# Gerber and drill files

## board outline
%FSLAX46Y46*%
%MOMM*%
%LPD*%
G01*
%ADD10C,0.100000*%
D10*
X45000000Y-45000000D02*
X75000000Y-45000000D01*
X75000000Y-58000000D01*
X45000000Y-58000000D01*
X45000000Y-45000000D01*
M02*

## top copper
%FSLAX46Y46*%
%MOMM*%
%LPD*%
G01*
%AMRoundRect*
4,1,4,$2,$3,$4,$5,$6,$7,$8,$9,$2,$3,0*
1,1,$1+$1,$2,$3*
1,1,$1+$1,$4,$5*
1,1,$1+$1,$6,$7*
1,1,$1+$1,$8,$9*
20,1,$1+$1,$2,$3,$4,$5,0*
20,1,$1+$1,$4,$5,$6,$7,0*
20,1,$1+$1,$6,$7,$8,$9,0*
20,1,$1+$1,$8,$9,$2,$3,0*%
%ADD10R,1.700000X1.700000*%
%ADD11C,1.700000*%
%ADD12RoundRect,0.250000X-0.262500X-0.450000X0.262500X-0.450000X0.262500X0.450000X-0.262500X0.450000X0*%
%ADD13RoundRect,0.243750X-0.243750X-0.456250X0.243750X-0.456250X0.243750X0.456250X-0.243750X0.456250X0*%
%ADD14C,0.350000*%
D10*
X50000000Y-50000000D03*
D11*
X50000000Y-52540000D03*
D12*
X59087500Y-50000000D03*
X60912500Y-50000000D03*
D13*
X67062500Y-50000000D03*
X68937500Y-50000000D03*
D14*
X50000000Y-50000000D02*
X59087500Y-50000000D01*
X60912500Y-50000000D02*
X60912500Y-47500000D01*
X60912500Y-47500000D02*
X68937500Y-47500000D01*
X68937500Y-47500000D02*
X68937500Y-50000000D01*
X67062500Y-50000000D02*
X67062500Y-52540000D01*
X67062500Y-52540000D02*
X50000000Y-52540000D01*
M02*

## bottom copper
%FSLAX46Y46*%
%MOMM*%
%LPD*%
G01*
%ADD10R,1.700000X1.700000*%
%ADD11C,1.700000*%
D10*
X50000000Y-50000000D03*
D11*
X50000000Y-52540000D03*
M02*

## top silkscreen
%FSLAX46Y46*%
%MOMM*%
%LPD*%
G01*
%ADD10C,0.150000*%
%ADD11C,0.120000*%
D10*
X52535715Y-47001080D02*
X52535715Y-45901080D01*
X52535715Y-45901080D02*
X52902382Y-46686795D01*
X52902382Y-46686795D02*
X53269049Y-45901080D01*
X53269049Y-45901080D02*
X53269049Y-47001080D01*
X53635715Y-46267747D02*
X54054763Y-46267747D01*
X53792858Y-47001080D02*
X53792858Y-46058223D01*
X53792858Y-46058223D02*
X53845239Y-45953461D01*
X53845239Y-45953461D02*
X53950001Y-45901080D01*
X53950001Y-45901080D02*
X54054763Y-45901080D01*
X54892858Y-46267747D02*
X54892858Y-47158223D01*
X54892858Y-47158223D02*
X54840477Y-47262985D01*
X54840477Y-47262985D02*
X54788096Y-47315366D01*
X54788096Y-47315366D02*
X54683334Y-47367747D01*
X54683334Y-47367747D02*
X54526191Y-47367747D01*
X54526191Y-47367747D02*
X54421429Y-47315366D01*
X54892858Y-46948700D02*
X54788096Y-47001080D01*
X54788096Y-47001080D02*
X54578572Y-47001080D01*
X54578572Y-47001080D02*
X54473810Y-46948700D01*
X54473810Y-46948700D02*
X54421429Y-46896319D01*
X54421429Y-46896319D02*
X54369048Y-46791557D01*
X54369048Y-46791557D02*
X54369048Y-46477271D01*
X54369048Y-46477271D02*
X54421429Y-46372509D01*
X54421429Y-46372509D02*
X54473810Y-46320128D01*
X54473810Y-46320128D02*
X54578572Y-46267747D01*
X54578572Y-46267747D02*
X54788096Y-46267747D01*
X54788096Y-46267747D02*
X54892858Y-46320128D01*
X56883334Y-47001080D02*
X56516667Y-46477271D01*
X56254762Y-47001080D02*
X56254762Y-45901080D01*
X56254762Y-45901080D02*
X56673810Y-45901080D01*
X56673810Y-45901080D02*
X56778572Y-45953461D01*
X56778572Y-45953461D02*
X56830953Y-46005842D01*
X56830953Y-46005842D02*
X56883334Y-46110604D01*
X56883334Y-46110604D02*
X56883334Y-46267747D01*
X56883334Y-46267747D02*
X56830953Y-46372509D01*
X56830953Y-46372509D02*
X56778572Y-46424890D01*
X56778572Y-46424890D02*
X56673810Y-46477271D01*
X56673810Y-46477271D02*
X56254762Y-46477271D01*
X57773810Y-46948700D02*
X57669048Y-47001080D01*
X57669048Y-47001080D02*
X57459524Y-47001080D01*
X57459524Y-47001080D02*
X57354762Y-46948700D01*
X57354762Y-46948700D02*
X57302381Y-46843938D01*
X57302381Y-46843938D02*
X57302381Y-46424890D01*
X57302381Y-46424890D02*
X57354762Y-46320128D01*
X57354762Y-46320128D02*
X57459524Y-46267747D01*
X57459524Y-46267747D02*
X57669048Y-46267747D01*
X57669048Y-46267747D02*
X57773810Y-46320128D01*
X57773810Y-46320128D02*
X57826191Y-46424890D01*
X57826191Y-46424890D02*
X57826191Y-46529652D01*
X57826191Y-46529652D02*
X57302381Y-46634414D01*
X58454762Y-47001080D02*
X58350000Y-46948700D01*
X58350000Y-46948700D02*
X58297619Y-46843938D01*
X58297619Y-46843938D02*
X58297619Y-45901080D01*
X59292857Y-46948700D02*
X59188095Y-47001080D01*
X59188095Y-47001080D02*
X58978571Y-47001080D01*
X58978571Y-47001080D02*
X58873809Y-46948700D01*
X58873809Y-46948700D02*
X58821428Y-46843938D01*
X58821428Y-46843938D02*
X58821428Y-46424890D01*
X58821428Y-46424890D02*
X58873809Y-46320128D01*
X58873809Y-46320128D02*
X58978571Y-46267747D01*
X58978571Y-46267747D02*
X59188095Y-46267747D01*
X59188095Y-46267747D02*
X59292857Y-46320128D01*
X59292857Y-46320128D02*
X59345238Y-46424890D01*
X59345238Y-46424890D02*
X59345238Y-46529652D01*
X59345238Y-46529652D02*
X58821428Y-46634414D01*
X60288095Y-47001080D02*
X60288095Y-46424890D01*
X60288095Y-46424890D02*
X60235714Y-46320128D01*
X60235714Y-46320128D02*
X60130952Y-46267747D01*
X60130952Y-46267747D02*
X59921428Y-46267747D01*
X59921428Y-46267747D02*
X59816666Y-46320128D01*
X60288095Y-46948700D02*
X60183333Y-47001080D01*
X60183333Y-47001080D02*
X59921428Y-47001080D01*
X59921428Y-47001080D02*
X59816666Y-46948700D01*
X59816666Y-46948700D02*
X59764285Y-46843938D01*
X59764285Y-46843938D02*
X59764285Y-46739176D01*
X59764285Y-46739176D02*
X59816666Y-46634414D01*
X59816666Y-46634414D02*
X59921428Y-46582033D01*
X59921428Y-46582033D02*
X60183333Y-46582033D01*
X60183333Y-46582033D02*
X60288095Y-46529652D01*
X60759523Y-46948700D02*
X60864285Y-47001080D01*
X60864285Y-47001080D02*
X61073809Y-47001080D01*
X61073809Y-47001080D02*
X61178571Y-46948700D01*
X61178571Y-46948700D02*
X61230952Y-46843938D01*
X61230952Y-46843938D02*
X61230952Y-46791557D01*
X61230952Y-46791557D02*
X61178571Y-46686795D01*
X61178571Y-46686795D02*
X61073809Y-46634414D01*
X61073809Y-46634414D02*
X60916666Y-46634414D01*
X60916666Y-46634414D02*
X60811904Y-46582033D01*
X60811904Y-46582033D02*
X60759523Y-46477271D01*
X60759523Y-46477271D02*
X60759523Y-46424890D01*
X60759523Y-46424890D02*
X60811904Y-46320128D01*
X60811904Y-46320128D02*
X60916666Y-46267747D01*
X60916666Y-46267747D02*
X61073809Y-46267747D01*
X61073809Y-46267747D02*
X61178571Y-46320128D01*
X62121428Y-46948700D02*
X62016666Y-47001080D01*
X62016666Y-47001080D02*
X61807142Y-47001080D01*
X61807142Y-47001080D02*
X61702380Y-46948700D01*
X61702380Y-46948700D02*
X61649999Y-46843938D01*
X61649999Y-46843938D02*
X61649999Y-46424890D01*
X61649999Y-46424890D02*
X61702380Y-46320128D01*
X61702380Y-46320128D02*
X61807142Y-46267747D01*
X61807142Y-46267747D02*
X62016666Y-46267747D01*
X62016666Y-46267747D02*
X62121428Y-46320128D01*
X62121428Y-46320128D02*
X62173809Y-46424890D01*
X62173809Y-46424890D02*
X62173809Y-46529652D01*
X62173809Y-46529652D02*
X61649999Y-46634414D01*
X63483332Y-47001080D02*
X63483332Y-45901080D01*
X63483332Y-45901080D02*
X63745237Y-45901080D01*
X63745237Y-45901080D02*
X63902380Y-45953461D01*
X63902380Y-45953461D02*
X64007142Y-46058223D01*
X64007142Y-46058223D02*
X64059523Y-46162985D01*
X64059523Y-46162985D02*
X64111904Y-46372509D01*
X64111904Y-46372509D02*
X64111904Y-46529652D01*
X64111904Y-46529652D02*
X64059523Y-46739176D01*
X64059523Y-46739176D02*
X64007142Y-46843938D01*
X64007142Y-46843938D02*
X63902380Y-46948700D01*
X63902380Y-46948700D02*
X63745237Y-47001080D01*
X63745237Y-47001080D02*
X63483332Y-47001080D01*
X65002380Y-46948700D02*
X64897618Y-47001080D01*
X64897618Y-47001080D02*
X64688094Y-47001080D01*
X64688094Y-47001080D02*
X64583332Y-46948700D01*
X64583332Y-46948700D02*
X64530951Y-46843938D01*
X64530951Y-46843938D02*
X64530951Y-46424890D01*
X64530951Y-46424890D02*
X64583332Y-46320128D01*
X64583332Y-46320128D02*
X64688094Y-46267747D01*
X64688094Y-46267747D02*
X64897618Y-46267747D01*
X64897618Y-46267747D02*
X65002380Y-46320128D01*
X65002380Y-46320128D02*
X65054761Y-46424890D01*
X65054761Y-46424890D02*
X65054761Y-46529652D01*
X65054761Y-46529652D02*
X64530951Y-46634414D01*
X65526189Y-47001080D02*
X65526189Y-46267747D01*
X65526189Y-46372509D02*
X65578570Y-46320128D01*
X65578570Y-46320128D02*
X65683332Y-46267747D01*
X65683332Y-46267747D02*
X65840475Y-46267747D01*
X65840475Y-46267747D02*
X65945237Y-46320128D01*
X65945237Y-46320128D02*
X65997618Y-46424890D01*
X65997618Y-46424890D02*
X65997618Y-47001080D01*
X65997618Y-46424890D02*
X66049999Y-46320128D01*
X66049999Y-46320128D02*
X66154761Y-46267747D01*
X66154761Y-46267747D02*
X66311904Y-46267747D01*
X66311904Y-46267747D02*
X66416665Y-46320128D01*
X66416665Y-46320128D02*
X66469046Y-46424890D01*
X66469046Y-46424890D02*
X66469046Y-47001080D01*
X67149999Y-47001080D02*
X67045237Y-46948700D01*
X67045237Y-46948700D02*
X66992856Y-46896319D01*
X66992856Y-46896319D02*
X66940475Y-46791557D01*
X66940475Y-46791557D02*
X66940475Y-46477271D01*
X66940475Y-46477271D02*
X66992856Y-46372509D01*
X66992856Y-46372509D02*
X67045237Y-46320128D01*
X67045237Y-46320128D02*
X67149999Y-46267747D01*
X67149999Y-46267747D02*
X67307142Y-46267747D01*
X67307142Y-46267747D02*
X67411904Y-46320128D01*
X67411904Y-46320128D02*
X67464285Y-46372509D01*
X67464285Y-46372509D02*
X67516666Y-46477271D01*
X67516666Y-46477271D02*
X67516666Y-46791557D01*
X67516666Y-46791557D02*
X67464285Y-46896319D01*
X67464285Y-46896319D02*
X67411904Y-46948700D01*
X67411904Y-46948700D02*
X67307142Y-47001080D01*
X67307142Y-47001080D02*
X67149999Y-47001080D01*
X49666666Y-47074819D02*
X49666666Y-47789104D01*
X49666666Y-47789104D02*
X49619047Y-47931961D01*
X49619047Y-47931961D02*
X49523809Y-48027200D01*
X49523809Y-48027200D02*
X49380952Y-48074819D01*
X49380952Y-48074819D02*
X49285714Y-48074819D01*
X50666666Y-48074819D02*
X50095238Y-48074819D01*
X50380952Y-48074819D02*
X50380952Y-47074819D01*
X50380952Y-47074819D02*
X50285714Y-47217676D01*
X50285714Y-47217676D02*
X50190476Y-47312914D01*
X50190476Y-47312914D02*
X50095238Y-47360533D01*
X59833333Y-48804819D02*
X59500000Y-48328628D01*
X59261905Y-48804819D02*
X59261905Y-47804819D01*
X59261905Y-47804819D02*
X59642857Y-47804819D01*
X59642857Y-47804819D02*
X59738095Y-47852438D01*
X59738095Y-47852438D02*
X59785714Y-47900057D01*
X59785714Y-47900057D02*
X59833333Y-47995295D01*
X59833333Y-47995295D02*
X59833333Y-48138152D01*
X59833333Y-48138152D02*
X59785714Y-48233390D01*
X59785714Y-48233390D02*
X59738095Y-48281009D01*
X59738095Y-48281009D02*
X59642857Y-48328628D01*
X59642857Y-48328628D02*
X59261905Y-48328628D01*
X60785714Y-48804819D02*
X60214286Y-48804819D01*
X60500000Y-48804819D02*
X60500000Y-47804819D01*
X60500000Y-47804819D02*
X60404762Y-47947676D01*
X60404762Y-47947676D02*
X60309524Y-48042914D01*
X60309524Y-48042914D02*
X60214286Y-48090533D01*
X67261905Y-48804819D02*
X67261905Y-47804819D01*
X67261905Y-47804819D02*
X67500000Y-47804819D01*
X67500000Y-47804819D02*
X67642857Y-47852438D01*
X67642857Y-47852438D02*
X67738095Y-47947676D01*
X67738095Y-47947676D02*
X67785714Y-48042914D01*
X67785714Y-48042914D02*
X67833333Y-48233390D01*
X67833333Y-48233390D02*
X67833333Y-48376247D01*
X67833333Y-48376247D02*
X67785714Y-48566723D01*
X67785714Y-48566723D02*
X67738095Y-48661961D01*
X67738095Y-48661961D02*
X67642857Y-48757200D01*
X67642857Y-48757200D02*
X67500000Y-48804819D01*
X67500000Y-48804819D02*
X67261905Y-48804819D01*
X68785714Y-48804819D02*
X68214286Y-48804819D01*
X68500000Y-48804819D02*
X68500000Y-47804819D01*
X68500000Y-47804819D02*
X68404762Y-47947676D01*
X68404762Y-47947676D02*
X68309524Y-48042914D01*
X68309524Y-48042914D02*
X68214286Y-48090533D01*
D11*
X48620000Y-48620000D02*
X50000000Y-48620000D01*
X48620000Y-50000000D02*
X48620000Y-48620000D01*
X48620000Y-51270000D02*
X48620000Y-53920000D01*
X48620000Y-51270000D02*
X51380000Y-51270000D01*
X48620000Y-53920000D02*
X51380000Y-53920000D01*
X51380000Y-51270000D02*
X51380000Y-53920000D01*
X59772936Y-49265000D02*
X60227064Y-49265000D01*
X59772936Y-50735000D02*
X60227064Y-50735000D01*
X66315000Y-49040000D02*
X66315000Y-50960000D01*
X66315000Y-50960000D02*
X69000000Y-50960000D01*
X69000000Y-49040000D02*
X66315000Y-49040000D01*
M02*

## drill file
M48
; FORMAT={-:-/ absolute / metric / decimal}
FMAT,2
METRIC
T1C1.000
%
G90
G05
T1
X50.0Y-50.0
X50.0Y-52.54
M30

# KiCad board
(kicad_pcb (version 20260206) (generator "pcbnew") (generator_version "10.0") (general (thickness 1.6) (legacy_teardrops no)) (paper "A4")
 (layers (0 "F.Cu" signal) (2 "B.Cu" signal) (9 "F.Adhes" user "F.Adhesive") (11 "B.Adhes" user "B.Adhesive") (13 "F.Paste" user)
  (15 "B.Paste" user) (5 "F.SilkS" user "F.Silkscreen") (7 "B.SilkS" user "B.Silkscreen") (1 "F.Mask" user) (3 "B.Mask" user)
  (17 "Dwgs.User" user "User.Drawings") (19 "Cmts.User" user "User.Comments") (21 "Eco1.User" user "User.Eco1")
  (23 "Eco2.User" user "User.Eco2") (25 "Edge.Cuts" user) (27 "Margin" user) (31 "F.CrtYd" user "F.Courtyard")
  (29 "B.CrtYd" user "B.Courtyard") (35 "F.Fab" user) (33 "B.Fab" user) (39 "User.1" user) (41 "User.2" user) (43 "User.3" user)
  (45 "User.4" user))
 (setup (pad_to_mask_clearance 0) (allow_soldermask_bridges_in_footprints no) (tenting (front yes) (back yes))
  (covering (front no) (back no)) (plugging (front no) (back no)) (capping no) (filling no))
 (gr_rect (start 45 45) (end 75 58) (stroke (width 0.1) (type solid)) (fill no) (layer "Edge.Cuts"))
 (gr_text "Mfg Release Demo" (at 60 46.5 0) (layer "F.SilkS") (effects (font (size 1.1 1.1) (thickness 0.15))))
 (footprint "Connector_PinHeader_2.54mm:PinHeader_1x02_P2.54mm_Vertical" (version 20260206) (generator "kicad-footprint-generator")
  (layer "F.Cu") (at 50 50 0)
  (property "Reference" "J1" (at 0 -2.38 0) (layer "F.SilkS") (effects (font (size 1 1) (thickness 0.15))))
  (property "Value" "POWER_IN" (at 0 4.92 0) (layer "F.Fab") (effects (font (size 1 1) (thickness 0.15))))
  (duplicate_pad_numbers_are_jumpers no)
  (fp_line (start -1.38 -1.38) (end 0 -1.38) (stroke (width 0.12) (type solid)) (layer "F.SilkS"))
  (fp_line (start -1.38 0) (end -1.38 -1.38) (stroke (width 0.12) (type solid)) (layer "F.SilkS"))
  (fp_line (start -1.38 1.27) (end -1.38 3.92) (stroke (width 0.12) (type solid)) (layer "F.SilkS"))
  (fp_line (start -1.38 1.27) (end 1.38 1.27) (stroke (width 0.12) (type solid)) (layer "F.SilkS"))
  (fp_line (start -1.38 3.92) (end 1.38 3.92) (stroke (width 0.12) (type solid)) (layer "F.SilkS"))
  (fp_line (start 1.38 1.27) (end 1.38 3.92) (stroke (width 0.12) (type solid)) (layer "F.SilkS"))
  (pad "1" thru_hole rect (at 0 0) (size 1.7 1.7) (drill 1) (layers "*.Cu" "*.Mask") (remove_unused_layers no) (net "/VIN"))
  (pad "2" thru_hole circle (at 0 2.54) (size 1.7 1.7) (drill 1) (layers "*.Cu" "*.Mask") (remove_unused_layers no) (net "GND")))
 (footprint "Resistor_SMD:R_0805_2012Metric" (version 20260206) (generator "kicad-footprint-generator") (layer "F.Cu") (at 60 50 0)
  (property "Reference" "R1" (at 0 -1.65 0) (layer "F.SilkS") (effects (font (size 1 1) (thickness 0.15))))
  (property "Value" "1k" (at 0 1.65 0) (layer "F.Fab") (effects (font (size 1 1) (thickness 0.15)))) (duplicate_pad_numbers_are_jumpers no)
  (fp_line (start -0.227064 -0.735) (end 0.227064 -0.735) (stroke (width 0.12) (type solid)) (layer "F.SilkS"))
  (fp_line (start -0.227064 0.735) (end 0.227064 0.735) (stroke (width 0.12) (type solid)) (layer "F.SilkS"))
  (pad "1" smd roundrect (at -0.9125 0) (size 1.025 1.4) (layers "F.Cu" "F.Mask" "F.Paste") (roundrect_rratio 0.243902) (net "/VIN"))
  (pad "2" smd roundrect (at 0.9125 0) (size 1.025 1.4) (layers "F.Cu" "F.Mask" "F.Paste") (roundrect_rratio 0.243902) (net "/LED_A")))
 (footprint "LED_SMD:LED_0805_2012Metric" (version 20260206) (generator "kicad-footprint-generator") (layer "F.Cu") (at 68 50 0)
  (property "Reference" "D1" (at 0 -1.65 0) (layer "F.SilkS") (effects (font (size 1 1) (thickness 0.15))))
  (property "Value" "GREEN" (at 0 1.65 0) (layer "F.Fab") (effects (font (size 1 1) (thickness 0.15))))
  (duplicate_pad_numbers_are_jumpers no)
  (fp_line (start -1.685 -0.96) (end -1.685 0.96) (stroke (width 0.12) (type solid)) (layer "F.SilkS"))
  (fp_line (start -1.685 0.96) (end 1 0.96) (stroke (width 0.12) (type solid)) (layer "F.SilkS"))
  (fp_line (start 1 -0.96) (end -1.685 -0.96) (stroke (width 0.12) (type solid)) (layer "F.SilkS"))
  (pad "1" smd roundrect (at -0.9375 0) (size 0.975 1.4) (layers "F.Cu" "F.Mask" "F.Paste") (roundrect_rratio 0.25) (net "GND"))
  (pad "2" smd roundrect (at 0.9375 0) (size 0.975 1.4) (layers "F.Cu" "F.Mask" "F.Paste") (roundrect_rratio 0.25) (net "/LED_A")))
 (segment (start 50 50) (end 59.0875 50) (width 0.35) (layer "F.Cu") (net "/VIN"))
 (segment (start 60.9125 50) (end 60.9125 47.5) (width 0.35) (layer "F.Cu") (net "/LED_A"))
 (segment (start 60.9125 47.5) (end 68.9375 47.5) (width 0.35) (layer "F.Cu") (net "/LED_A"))
 (segment (start 68.9375 47.5) (end 68.9375 50) (width 0.35) (layer "F.Cu") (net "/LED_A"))
 (segment (start 67.0625 50) (end 67.0625 52.54) (width 0.35) (layer "F.Cu") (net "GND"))
 (segment (start 67.0625 52.54) (end 50 52.54) (width 0.35) (layer "F.Cu") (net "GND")))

